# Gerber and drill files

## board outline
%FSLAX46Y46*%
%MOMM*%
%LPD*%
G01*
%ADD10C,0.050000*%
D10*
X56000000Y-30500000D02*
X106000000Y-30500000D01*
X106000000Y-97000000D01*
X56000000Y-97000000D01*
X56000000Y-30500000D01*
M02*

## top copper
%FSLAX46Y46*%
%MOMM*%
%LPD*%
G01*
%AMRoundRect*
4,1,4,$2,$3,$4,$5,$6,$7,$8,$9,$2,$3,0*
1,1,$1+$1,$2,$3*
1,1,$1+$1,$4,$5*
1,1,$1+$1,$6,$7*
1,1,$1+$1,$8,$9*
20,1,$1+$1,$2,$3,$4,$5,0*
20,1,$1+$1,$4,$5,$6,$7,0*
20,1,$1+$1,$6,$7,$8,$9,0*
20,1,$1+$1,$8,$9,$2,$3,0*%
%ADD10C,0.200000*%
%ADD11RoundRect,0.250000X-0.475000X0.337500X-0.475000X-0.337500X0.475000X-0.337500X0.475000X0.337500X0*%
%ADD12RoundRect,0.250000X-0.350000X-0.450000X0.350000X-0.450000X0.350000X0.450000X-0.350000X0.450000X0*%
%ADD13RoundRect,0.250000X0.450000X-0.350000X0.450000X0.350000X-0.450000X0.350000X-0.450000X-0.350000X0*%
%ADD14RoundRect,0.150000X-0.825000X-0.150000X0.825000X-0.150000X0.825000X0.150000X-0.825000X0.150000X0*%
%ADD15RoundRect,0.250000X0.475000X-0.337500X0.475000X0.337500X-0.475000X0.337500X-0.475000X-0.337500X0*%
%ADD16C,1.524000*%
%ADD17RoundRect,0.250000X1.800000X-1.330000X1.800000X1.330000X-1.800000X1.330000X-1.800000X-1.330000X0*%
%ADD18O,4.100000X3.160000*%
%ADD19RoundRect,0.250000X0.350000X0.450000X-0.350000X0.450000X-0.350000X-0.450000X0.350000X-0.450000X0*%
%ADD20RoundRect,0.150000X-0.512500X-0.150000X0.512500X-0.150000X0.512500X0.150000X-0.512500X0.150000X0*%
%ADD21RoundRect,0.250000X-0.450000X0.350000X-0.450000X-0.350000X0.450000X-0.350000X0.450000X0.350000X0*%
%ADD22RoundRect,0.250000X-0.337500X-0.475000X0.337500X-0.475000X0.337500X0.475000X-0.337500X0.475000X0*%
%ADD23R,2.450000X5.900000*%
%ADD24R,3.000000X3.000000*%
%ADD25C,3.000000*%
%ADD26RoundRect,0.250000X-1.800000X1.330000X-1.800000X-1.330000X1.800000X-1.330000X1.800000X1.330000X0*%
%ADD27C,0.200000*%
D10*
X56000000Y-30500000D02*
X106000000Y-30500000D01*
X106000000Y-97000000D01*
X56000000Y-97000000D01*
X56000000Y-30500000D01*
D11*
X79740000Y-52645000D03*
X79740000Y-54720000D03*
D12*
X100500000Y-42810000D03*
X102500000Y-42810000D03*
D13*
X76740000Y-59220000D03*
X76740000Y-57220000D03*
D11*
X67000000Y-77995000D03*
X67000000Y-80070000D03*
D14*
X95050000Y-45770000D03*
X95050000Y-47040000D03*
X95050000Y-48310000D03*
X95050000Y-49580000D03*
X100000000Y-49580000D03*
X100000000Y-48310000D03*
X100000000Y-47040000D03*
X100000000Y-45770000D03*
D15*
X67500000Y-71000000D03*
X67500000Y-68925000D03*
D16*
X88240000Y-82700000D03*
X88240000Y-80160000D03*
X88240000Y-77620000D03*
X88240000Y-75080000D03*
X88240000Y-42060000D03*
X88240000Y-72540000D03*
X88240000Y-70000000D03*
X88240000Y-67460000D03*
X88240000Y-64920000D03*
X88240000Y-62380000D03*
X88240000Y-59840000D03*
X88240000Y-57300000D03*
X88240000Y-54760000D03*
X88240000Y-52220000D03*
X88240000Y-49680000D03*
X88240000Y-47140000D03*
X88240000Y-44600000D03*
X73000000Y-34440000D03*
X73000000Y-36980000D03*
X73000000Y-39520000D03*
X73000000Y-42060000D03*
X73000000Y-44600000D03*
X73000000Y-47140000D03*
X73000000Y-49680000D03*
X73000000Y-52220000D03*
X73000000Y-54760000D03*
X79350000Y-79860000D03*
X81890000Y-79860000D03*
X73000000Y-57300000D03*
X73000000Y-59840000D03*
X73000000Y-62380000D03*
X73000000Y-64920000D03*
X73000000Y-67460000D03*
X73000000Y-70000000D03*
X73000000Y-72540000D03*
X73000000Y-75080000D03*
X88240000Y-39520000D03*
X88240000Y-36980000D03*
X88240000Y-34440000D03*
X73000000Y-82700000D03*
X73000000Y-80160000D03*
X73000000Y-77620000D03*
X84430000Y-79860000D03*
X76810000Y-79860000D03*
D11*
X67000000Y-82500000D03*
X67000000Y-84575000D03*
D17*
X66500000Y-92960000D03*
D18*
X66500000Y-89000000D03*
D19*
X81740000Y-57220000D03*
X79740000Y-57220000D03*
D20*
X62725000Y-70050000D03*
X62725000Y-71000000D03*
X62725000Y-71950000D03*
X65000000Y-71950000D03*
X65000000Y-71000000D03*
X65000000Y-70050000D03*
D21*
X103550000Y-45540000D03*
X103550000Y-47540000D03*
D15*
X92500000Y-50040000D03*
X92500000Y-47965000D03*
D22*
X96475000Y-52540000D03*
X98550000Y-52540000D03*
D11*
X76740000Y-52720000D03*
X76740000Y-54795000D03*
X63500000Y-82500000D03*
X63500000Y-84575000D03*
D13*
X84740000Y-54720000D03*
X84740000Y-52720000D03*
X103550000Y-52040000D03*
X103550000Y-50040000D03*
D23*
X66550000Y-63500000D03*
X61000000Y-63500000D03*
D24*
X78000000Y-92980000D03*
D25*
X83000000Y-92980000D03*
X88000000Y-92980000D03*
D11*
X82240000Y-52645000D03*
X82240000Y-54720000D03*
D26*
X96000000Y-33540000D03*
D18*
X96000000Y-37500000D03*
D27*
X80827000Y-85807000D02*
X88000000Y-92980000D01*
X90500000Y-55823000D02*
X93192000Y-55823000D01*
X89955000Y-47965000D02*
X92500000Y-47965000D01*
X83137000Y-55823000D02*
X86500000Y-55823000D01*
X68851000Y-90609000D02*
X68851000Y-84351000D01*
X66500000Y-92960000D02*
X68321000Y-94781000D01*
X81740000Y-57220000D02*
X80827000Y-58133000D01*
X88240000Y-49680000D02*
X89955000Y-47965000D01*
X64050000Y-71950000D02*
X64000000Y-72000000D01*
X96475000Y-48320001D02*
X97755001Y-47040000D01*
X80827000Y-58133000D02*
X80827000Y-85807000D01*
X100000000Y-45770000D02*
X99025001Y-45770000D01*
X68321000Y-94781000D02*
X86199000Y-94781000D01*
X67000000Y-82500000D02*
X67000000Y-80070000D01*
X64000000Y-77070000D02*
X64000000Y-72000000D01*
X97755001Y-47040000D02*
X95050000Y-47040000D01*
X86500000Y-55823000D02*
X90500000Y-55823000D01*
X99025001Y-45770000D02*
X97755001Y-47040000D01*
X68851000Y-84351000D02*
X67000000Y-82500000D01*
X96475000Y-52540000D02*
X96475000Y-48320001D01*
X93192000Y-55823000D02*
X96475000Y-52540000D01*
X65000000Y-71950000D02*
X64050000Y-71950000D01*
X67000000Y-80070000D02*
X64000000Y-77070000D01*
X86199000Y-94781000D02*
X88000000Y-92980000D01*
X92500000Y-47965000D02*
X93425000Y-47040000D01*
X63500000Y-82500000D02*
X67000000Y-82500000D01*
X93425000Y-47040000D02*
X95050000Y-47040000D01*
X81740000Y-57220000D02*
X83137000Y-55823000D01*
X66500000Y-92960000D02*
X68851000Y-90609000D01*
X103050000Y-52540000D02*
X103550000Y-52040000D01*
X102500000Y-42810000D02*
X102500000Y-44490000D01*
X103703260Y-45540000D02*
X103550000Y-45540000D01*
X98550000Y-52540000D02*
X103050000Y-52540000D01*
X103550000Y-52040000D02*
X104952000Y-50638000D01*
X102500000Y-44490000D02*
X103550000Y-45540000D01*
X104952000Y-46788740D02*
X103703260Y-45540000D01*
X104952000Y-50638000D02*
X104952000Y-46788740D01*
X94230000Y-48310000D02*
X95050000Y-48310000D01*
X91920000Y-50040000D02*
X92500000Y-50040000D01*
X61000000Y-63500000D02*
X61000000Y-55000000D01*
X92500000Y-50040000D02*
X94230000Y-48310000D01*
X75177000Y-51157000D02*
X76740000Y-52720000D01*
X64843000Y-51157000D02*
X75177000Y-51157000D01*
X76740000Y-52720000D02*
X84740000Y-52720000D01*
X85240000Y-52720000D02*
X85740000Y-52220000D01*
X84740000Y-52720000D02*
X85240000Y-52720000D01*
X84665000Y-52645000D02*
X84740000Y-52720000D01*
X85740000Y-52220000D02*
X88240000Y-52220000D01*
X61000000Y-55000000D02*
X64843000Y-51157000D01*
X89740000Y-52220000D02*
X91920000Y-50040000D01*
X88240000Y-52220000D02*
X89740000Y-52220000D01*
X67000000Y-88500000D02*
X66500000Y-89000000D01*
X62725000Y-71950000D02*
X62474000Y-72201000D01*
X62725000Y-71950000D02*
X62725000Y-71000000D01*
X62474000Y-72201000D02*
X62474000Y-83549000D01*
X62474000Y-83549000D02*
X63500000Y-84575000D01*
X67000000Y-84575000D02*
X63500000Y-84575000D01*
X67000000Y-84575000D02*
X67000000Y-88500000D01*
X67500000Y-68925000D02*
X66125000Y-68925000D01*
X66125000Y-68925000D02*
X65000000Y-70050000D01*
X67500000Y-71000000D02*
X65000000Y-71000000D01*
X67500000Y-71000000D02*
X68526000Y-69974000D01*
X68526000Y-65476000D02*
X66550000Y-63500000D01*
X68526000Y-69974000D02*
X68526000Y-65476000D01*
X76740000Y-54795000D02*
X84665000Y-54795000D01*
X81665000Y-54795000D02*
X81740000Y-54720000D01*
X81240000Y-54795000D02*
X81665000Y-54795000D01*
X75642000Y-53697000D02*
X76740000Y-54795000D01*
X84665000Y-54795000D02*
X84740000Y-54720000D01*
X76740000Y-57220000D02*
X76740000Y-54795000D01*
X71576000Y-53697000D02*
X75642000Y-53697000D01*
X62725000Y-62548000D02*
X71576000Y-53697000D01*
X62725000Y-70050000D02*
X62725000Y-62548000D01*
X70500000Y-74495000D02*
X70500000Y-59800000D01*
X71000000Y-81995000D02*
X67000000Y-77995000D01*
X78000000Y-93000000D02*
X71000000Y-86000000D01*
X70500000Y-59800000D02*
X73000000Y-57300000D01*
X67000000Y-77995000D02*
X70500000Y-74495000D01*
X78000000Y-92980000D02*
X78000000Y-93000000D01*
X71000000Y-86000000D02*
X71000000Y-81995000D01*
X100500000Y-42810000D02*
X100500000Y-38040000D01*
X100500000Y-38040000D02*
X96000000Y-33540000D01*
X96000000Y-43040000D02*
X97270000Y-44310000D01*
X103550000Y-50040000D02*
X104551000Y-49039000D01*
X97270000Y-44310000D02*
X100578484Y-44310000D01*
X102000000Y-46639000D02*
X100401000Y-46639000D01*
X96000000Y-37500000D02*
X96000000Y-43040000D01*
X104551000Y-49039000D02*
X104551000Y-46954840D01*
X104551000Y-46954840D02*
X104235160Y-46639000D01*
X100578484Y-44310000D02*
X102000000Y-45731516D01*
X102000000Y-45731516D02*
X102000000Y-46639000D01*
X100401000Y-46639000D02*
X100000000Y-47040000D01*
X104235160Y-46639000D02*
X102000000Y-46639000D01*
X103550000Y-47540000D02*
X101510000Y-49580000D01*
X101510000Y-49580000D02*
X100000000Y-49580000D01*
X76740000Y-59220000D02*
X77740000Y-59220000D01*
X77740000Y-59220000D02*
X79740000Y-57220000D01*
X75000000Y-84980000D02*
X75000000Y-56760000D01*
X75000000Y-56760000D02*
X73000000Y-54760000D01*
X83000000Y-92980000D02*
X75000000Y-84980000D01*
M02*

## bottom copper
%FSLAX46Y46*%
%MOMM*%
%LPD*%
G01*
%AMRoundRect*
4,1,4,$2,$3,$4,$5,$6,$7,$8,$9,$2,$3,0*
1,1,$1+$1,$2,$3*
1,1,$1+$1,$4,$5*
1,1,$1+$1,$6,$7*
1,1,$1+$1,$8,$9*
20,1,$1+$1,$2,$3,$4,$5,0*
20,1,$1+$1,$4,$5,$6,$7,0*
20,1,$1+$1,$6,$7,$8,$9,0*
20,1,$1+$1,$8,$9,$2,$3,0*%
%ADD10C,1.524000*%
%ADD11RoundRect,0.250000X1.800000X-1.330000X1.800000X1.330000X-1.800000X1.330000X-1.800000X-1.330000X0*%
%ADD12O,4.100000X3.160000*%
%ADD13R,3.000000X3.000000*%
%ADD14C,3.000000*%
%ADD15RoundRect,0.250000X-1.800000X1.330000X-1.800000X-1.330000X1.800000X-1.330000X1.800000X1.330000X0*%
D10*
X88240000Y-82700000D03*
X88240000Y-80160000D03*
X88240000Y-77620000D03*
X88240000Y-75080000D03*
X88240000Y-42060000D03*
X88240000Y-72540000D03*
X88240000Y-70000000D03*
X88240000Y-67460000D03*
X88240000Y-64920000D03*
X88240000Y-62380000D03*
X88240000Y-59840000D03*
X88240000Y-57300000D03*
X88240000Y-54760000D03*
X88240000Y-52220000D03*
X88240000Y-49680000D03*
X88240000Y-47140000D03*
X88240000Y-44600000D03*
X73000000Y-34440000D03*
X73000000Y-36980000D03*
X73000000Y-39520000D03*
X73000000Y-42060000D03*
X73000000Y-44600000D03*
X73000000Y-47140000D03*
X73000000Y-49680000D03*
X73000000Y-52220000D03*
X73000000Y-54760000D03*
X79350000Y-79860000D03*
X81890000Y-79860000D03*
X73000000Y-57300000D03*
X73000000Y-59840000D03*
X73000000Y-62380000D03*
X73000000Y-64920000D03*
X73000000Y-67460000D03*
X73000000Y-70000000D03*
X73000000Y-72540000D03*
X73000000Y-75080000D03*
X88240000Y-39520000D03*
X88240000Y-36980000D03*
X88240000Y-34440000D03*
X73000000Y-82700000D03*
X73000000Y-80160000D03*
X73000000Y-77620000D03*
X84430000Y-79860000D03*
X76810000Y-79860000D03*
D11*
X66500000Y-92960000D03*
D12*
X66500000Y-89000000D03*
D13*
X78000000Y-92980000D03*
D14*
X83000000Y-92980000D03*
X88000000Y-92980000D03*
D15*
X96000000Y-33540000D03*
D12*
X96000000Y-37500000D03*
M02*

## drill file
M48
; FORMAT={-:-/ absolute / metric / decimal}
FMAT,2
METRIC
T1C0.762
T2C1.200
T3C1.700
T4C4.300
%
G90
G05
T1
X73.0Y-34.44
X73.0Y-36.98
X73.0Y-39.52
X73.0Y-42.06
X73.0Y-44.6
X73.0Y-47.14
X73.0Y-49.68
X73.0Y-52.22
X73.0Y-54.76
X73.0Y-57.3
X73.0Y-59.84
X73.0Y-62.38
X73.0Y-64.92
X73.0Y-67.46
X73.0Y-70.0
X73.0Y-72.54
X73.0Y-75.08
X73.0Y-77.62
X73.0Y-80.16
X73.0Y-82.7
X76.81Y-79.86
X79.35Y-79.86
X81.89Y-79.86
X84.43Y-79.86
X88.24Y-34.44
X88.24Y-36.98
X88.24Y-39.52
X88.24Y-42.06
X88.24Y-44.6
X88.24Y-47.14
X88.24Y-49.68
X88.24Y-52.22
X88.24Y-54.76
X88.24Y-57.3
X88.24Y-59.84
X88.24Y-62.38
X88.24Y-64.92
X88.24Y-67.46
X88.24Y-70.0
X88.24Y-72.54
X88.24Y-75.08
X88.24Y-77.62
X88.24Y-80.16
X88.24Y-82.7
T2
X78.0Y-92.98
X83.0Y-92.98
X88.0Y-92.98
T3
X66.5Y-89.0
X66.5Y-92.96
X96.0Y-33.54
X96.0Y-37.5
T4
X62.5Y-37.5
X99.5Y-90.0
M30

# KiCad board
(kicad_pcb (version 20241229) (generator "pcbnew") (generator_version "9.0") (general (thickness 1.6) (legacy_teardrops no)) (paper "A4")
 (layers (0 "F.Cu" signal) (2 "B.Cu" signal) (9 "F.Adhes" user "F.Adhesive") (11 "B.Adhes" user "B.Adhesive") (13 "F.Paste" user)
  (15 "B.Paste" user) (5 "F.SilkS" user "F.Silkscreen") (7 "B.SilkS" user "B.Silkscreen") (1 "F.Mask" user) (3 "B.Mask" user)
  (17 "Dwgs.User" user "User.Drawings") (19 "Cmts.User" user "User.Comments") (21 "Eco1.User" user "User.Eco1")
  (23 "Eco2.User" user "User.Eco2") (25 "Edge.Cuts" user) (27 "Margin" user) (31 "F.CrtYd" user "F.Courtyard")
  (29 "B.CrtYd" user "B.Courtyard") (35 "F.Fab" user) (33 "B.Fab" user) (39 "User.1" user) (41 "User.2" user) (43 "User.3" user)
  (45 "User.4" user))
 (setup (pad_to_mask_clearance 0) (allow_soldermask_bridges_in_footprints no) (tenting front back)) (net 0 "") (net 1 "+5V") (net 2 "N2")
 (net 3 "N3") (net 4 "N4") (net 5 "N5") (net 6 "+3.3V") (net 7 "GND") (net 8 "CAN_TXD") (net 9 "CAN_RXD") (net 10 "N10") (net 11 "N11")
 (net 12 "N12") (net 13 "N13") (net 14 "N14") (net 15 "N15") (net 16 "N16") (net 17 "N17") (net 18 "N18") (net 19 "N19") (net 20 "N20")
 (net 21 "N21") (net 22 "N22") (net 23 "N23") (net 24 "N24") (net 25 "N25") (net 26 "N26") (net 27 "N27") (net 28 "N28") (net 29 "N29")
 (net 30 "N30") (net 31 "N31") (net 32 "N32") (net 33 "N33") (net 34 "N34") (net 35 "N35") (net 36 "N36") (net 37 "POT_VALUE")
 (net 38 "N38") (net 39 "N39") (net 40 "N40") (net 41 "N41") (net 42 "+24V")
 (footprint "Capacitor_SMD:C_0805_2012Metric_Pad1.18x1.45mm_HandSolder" (layer "F.Cu") (at 79.74 53.6825 -90)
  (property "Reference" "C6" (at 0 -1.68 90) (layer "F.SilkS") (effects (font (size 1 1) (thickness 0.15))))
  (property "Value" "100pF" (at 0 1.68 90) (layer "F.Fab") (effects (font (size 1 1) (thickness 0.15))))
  (pad "1" smd roundrect (at -1.0375 0 270) (size 1.175 1.45) (layers "F.Cu" "F.Mask" "F.Paste") (roundrect_rratio 0.212766) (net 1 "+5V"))
  (pad "2" smd roundrect (at 1.0375 0 270) (size 1.175 1.45) (layers "F.Cu" "F.Mask" "F.Paste") (roundrect_rratio 0.212766) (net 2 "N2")))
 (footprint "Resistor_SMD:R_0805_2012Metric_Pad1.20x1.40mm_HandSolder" (layer "F.Cu") (at 101.5 42.81)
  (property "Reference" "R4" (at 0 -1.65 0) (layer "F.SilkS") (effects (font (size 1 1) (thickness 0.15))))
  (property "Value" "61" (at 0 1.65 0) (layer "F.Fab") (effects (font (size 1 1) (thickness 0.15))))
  (pad "1" smd roundrect (at -1 0) (size 1.2 1.4) (layers "F.Cu" "F.Mask" "F.Paste") (roundrect_rratio 0.208333) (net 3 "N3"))
  (pad "2" smd roundrect (at 1 0) (size 1.2 1.4) (layers "F.Cu" "F.Mask" "F.Paste") (roundrect_rratio 0.208333) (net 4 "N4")))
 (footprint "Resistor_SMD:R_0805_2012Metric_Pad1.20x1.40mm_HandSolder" (layer "F.Cu") (at 76.74 58.22 90)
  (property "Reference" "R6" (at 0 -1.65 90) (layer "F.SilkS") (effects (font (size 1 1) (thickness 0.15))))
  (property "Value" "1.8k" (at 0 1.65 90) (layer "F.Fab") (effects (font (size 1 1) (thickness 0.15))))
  (pad "1" smd roundrect (at -1 0 90) (size 1.2 1.4) (layers "F.Cu" "F.Mask" "F.Paste") (roundrect_rratio 0.208333) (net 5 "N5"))
  (pad "2" smd roundrect (at 1 0 90) (size 1.2 1.4) (layers "F.Cu" "F.Mask" "F.Paste") (roundrect_rratio 0.208333) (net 2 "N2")))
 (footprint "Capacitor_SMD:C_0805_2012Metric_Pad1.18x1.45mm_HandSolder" (layer "F.Cu") (at 67 79.0325 -90)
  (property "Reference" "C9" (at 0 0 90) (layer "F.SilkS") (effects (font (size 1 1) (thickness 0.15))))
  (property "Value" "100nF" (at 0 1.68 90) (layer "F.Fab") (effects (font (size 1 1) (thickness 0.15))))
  (pad "1" smd roundrect (at -1.0375 0 270) (size 1.175 1.45) (layers "F.Cu" "F.Mask" "F.Paste") (roundrect_rratio 0.212766) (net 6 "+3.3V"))
  (pad "2" smd roundrect (at 1.0375 0 270) (size 1.175 1.45) (layers "F.Cu" "F.Mask" "F.Paste") (roundrect_rratio 0.212766) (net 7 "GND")))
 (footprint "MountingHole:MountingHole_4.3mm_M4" (layer "F.Cu") (at 62.5 37.5)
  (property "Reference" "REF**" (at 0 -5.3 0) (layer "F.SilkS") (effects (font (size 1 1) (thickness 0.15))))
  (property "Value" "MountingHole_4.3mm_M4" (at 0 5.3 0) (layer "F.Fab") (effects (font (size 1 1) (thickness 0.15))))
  (pad "" np_thru_hole circle (at 0 0) (size 4.3 4.3) (drill 4.3) (layers "*.Cu" "*.Mask")))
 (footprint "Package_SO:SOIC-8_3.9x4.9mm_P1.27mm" (layer "F.Cu") (at 97.525 47.675)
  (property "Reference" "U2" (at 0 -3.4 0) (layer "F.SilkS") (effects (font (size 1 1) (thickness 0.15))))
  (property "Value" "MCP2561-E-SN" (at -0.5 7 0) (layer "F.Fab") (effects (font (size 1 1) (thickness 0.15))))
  (pad "1" smd roundrect (at -2.475 -1.905) (size 1.95 0.6) (layers "F.Cu" "F.Mask" "F.Paste") (roundrect_rratio 0.25) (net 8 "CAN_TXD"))
  (pad "2" smd roundrect (at -2.475 -0.635) (size 1.95 0.6) (layers "F.Cu" "F.Mask" "F.Paste") (roundrect_rratio 0.25) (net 7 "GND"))
  (pad "3" smd roundrect (at -2.475 0.635) (size 1.95 0.6) (layers "F.Cu" "F.Mask" "F.Paste") (roundrect_rratio 0.25) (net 1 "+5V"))
  (pad "4" smd roundrect (at -2.475 1.905) (size 1.95 0.6) (layers "F.Cu" "F.Mask" "F.Paste") (roundrect_rratio 0.25) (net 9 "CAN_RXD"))
  (pad "5" smd roundrect (at 2.475 1.905) (size 1.95 0.6) (layers "F.Cu" "F.Mask" "F.Paste") (roundrect_rratio 0.25) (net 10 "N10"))
  (pad "6" smd roundrect (at 2.475 0.635) (size 1.95 0.6) (layers "F.Cu" "F.Mask" "F.Paste") (roundrect_rratio 0.25) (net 3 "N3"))
  (pad "7" smd roundrect (at 2.475 -0.635) (size 1.95 0.6) (layers "F.Cu" "F.Mask" "F.Paste") (roundrect_rratio 0.25) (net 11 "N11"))
  (pad "8" smd roundrect (at 2.475 -1.905) (size 1.95 0.6) (layers "F.Cu" "F.Mask" "F.Paste") (roundrect_rratio 0.25) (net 7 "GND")))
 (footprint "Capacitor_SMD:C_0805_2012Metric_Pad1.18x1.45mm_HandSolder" (layer "F.Cu") (at 67.5 69.9625 90)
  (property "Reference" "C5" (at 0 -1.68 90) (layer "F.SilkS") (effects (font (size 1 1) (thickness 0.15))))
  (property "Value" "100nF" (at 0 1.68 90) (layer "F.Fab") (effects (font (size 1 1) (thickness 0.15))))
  (pad "1" smd roundrect (at -1.0375 0 90) (size 1.175 1.45) (layers "F.Cu" "F.Mask" "F.Paste") (roundrect_rratio 0.212766) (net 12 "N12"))
  (pad "2" smd roundrect (at 1.0375 0 90) (size 1.175 1.45) (layers "F.Cu" "F.Mask" "F.Paste") (roundrect_rratio 0.212766) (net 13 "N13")))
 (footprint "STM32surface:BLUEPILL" (layer "F.Cu") (at 80.62 61.11 180)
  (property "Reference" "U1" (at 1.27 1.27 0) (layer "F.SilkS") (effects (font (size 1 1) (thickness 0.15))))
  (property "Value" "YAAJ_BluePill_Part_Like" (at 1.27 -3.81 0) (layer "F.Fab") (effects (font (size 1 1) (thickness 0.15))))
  (pad "1" thru_hole circle (at -7.62 -21.59 180) (size 1.524 1.524) (drill 0.762) (layers "*.Cu" "*.Mask") (remove_unused_layers no)
   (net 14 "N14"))
  (pad "2" thru_hole circle (at -7.62 -19.05 180) (size 1.524 1.524) (drill 0.762) (layers "*.Cu" "*.Mask") (remove_unused_layers no)
   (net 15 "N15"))
  (pad "3" thru_hole circle (at -7.62 -16.51 180) (size 1.524 1.524) (drill 0.762) (layers "*.Cu" "*.Mask") (remove_unused_layers no)
   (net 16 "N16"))
  (pad "4" thru_hole circle (at -7.62 -13.97 180) (size 1.524 1.524) (drill 0.762) (layers "*.Cu" "*.Mask") (remove_unused_layers no)
   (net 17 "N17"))
  (pad "7" thru_hole circle (at -7.62 19.05 180) (size 1.524 1.524) (drill 0.762) (layers "*.Cu" "*.Mask") (remove_unused_layers no)
   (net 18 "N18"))
  (pad "10" thru_hole circle (at -7.62 -11.43 180) (size 1.524 1.524) (drill 0.762) (layers "*.Cu" "*.Mask") (remove_unused_layers no)
   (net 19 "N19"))
  (pad "11" thru_hole circle (at -7.62 -8.89 180) (size 1.524 1.524) (drill 0.762) (layers "*.Cu" "*.Mask") (remove_unused_layers no)
   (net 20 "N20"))
  (pad "12" thru_hole circle (at -7.62 -6.35 180) (size 1.524 1.524) (drill 0.762) (layers "*.Cu" "*.Mask") (remove_unused_layers no)
   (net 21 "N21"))
  (pad "13" thru_hole circle (at -7.62 -3.81 180) (size 1.524 1.524) (drill 0.762) (layers "*.Cu" "*.Mask") (remove_unused_layers no)
   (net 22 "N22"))
  (pad "14" thru_hole circle (at -7.62 -1.27 180) (size 1.524 1.524) (drill 0.762) (layers "*.Cu" "*.Mask") (remove_unused_layers no)
   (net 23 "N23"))
  (pad "15" thru_hole circle (at -7.62 1.27 180) (size 1.524 1.524) (drill 0.762) (layers "*.Cu" "*.Mask") (remove_unused_layers no)
   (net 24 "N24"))
  (pad "16" thru_hole circle (at -7.62 3.81 180) (size 1.524 1.524) (drill 0.762) (layers "*.Cu" "*.Mask") (remove_unused_layers no)
   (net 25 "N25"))
  (pad "17" thru_hole circle (at -7.62 6.35 180) (size 1.524 1.524) (drill 0.762) (layers "*.Cu" "*.Mask") (remove_unused_layers no)
   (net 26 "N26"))
  (pad "18" thru_hole circle (at -7.62 8.89 180) (size 1.524 1.524) (drill 0.762) (layers "*.Cu" "*.Mask") (remove_unused_layers no)
   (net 1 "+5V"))
  (pad "19" thru_hole circle (at -7.62 11.43 180) (size 1.524 1.524) (drill 0.762) (layers "*.Cu" "*.Mask") (remove_unused_layers no)
   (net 7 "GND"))
  (pad "21" thru_hole circle (at -7.62 13.97 180) (size 1.524 1.524) (drill 0.762) (layers "*.Cu" "*.Mask") (remove_unused_layers no)
   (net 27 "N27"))
  (pad "22" thru_hole circle (at -7.62 16.51 180) (size 1.524 1.524) (drill 0.762) (layers "*.Cu" "*.Mask") (remove_unused_layers no)
   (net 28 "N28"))
  (pad "25" thru_hole circle (at 7.62 26.67 180) (size 1.524 1.524) (drill 0.762) (layers "*.Cu" "*.Mask") (remove_unused_layers no)
   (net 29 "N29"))
  (pad "26" thru_hole circle (at 7.62 24.13 180) (size 1.524 1.524) (drill 0.762) (layers "*.Cu" "*.Mask") (remove_unused_layers no)
   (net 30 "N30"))
  (pad "27" thru_hole circle (at 7.62 21.59 180) (size 1.524 1.524) (drill 0.762) (layers "*.Cu" "*.Mask") (remove_unused_layers no)
   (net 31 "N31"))
  (pad "28" thru_hole circle (at 7.62 19.05 180) (size 1.524 1.524) (drill 0.762) (layers "*.Cu" "*.Mask") (remove_unused_layers no)
   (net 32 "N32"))
  (pad "29" thru_hole circle (at 7.62 16.51 180) (size 1.524 1.524) (drill 0.762) (layers "*.Cu" "*.Mask") (remove_unused_layers no)
   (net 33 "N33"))
  (pad "30" thru_hole circle (at 7.62 13.97 180) (size 1.524 1.524) (drill 0.762) (layers "*.Cu" "*.Mask") (remove_unused_layers no)
   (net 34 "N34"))
  (pad "31" thru_hole circle (at 7.62 11.43 180) (size 1.524 1.524) (drill 0.762) (layers "*.Cu" "*.Mask") (remove_unused_layers no)
   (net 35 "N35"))
  (pad "32" thru_hole circle (at 7.62 8.89 180) (size 1.524 1.524) (drill 0.762) (layers "*.Cu" "*.Mask") (remove_unused_layers no)
   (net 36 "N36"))
  (pad "33" thru_hole circle (at 7.62 6.35 180) (size 1.524 1.524) (drill 0.762) (layers "*.Cu" "*.Mask") (remove_unused_layers no)
   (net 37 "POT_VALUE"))
  (pad "34" thru_hole circle (at 1.27 -18.75 180) (size 1.524 1.524) (drill 0.762) (layers "*.Cu" "*.Mask") (remove_unused_layers no)
   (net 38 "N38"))
  (pad "37" thru_hole circle (at -1.27 -18.75 180) (size 1.524 1.524) (drill 0.762) (layers "*.Cu" "*.Mask") (remove_unused_layers no)
   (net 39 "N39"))
  (pad "38" thru_hole circle (at 7.62 3.81 180) (size 1.524 1.524) (drill 0.762) (layers "*.Cu" "*.Mask") (remove_unused_layers no)
   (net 6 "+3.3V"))
  (pad "39" thru_hole circle (at 7.62 1.27 180) (size 1.524 1.524) (drill 0.762) (layers "*.Cu" "*.Mask") (remove_unused_layers no)
   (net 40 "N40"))
  (pad "40" thru_hole circle (at 7.62 -1.27 180) (size 1.524 1.524) (drill 0.762) (layers "*.Cu" "*.Mask") (remove_unused_layers no)
   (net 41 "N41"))
  (pad "41" thru_hole circle (at 7.62 -3.81 180) (size 1.524 1.524) (drill 0.762) (layers "*.Cu" "*.Mask") (remove_unused_layers no))
  (pad "42" thru_hole circle (at 7.62 -6.35 180) (size 1.524 1.524) (drill 0.762) (layers "*.Cu" "*.Mask") (remove_unused_layers no))
  (pad "43" thru_hole circle (at 7.62 -8.89 180) (size 1.524 1.524) (drill 0.762) (layers "*.Cu" "*.Mask") (remove_unused_layers no))
  (pad "45" thru_hole circle (at 7.62 -11.43 180) (size 1.524 1.524) (drill 0.762) (layers "*.Cu" "*.Mask") (remove_unused_layers no))
  (pad "46" thru_hole circle (at 7.62 -13.97 180) (size 1.524 1.524) (drill 0.762) (layers "*.Cu" "*.Mask") (remove_unused_layers no))
  (pad "70" thru_hole circle (at -7.62 21.59 180) (size 1.524 1.524) (drill 0.762) (layers "*.Cu" "*.Mask") (remove_unused_layers no))
  (pad "71" thru_hole circle (at -7.62 24.13 180) (size 1.524 1.524) (drill 0.762) (layers "*.Cu" "*.Mask") (remove_unused_layers no))
  (pad "72" thru_hole circle (at -7.62 26.67 180) (size 1.524 1.524) (drill 0.762) (layers "*.Cu" "*.Mask") (remove_unused_layers no))
  (pad "73" thru_hole circle (at 7.62 -21.59 180) (size 1.524 1.524) (drill 0.762) (layers "*.Cu" "*.Mask") (remove_unused_layers no))
  (pad "74" thru_hole circle (at 7.62 -19.05 180) (size 1.524 1.524) (drill 0.762) (layers "*.Cu" "*.Mask") (remove_unused_layers no))
  (pad "75" thru_hole circle (at 7.62 -16.51 180) (size 1.524 1.524) (drill 0.762) (layers "*.Cu" "*.Mask") (remove_unused_layers no))
  (pad "76" thru_hole circle (at -3.81 -18.75 180) (size 1.524 1.524) (drill 0.762) (layers "*.Cu" "*.Mask") (remove_unused_layers no))
  (pad "77" thru_hole circle (at 3.81 -18.75 180) (size 1.524 1.524) (drill 0.762) (layers "*.Cu" "*.Mask") (remove_unused_layers no)))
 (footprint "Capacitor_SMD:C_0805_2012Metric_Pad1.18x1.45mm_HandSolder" (layer "F.Cu") (at 67 83.5375 -90)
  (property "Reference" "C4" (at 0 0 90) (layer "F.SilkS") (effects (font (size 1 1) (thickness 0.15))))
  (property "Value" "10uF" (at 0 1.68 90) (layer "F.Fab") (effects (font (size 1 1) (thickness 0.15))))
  (pad "1" smd roundrect (at -1.0375 0 270) (size 1.175 1.45) (layers "F.Cu" "F.Mask" "F.Paste") (roundrect_rratio 0.212766) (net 7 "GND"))
  (pad "2" smd roundrect (at 1.0375 0 270) (size 1.175 1.45) (layers "F.Cu" "F.Mask" "F.Paste") (roundrect_rratio 0.212766) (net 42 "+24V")))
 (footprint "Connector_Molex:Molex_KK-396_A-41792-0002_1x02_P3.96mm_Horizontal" (layer "F.Cu") (at 66.5 92.96 90)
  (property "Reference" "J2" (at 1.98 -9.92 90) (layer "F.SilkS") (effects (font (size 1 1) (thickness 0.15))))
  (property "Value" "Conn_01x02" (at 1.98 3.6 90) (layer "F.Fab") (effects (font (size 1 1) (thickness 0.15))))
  (pad "1" thru_hole roundrect (at 0 0 90) (size 3.16 4.1) (drill 1.7) (layers "*.Cu" "*.Mask") (remove_unused_layers no)
   (roundrect_rratio 0.079114) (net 7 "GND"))
  (pad "2" thru_hole oval (at 3.96 0 90) (size 3.16 4.1) (drill 1.7) (layers "*.Cu" "*.Mask") (remove_unused_layers no) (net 42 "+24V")))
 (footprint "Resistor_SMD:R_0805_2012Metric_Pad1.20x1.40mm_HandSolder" (layer "F.Cu") (at 80.74 57.22 180)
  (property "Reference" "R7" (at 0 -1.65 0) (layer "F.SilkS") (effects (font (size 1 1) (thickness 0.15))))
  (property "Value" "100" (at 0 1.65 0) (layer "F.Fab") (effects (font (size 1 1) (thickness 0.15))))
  (pad "1" smd roundrect (at -1 0 180) (size 1.2 1.4) (layers "F.Cu" "F.Mask" "F.Paste") (roundrect_rratio 0.208333) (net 7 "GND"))
  (pad "2" smd roundrect (at 1 0 180) (size 1.2 1.4) (layers "F.Cu" "F.Mask" "F.Paste") (roundrect_rratio 0.208333) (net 5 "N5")))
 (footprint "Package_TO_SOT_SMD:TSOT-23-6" (layer "F.Cu") (at 63.8625 71)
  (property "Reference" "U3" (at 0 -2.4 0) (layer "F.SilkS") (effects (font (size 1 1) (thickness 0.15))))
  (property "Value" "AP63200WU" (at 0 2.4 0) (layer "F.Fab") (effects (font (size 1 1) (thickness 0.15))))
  (pad "1" smd roundrect (at -1.1375 -0.95) (size 1.325 0.6) (layers "F.Cu" "F.Mask" "F.Paste") (roundrect_rratio 0.25) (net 2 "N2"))
  (pad "2" smd roundrect (at -1.1375 0) (size 1.325 0.6) (layers "F.Cu" "F.Mask" "F.Paste") (roundrect_rratio 0.25) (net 42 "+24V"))
  (pad "3" smd roundrect (at -1.1375 0.95) (size 1.325 0.6) (layers "F.Cu" "F.Mask" "F.Paste") (roundrect_rratio 0.25) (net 42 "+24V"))
  (pad "4" smd roundrect (at 1.1375 0.95) (size 1.325 0.6) (layers "F.Cu" "F.Mask" "F.Paste") (roundrect_rratio 0.25) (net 7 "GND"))
  (pad "5" smd roundrect (at 1.1375 0) (size 1.325 0.6) (layers "F.Cu" "F.Mask" "F.Paste") (roundrect_rratio 0.25) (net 12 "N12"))
  (pad "6" smd roundrect (at 1.1375 -0.95) (size 1.325 0.6) (layers "F.Cu" "F.Mask" "F.Paste") (roundrect_rratio 0.25) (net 13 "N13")))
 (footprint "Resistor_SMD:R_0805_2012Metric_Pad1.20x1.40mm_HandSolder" (layer "F.Cu") (at 103.55 46.54 -90)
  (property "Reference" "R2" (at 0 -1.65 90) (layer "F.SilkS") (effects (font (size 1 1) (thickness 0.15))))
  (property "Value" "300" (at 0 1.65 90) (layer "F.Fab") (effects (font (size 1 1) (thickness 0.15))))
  (pad "1" smd roundrect (at -1 0 270) (size 1.2 1.4) (layers "F.Cu" "F.Mask" "F.Paste") (roundrect_rratio 0.208333) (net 4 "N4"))
  (pad "2" smd roundrect (at 1 0 270) (size 1.2 1.4) (layers "F.Cu" "F.Mask" "F.Paste") (roundrect_rratio 0.208333) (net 10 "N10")))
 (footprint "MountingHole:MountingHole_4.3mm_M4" (layer "F.Cu") (at 99.5 90)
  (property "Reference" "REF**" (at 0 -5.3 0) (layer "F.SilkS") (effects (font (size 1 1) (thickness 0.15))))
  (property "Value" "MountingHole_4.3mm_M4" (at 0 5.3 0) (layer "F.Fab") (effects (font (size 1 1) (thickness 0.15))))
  (pad "" np_thru_hole circle (at 0 0) (size 4.3 4.3) (drill 4.3) (layers "*.Cu" "*.Mask")))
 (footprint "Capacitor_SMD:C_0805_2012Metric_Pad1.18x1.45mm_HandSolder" (layer "F.Cu") (at 92.5 49.0025 90)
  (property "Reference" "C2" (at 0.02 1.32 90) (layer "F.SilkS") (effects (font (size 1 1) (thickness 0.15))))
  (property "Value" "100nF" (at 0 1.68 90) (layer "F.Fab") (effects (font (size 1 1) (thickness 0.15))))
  (pad "1" smd roundrect (at -1.0375 0 90) (size 1.175 1.45) (layers "F.Cu" "F.Mask" "F.Paste") (roundrect_rratio 0.212766) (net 1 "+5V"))
  (pad "2" smd roundrect (at 1.0375 0 90) (size 1.175 1.45) (layers "F.Cu" "F.Mask" "F.Paste") (roundrect_rratio 0.212766) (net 7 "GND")))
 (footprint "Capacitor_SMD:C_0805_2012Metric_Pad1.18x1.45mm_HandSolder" (layer "F.Cu") (at 97.5125 52.54)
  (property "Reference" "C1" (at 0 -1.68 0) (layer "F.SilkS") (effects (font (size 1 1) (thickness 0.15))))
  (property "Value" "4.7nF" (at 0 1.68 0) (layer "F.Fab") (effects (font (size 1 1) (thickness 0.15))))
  (pad "1" smd roundrect (at -1.0375 0) (size 1.175 1.45) (layers "F.Cu" "F.Mask" "F.Paste") (roundrect_rratio 0.212766) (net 7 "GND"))
  (pad "2" smd roundrect (at 1.0375 0) (size 1.175 1.45) (layers "F.Cu" "F.Mask" "F.Paste") (roundrect_rratio 0.212766) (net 4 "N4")))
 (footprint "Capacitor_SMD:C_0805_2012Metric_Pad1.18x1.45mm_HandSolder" (layer "F.Cu") (at 76.74 53.7575 -90)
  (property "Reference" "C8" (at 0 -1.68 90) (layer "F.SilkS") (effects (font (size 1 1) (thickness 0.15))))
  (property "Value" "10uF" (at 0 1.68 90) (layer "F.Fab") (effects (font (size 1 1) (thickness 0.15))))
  (pad "1" smd roundrect (at -1.0375 0 270) (size 1.175 1.45) (layers "F.Cu" "F.Mask" "F.Paste") (roundrect_rratio 0.212766) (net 1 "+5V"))
  (pad "2" smd roundrect (at 1.0375 0 270) (size 1.175 1.45) (layers "F.Cu" "F.Mask" "F.Paste") (roundrect_rratio 0.212766) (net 2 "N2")))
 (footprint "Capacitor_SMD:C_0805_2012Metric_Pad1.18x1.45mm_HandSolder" (layer "F.Cu") (at 63.5 83.5375 -90)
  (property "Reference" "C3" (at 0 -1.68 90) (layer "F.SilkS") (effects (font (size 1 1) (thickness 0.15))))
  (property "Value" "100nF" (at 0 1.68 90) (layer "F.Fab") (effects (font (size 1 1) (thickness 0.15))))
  (pad "1" smd roundrect (at -1.0375 0 270) (size 1.175 1.45) (layers "F.Cu" "F.Mask" "F.Paste") (roundrect_rratio 0.212766) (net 7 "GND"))
  (pad "2" smd roundrect (at 1.0375 0 270) (size 1.175 1.45) (layers "F.Cu" "F.Mask" "F.Paste") (roundrect_rratio 0.212766) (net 42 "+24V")))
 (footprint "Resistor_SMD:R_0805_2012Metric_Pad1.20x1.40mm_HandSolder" (layer "F.Cu") (at 84.74 53.72 90)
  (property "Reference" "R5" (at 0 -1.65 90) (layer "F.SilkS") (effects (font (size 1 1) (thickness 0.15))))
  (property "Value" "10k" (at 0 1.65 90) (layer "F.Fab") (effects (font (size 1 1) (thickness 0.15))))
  (pad "1" smd roundrect (at -1 0 90) (size 1.2 1.4) (layers "F.Cu" "F.Mask" "F.Paste") (roundrect_rratio 0.208333) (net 2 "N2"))
  (pad "2" smd roundrect (at 1 0 90) (size 1.2 1.4) (layers "F.Cu" "F.Mask" "F.Paste") (roundrect_rratio 0.208333) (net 1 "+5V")))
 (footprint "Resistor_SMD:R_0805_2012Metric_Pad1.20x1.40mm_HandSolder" (layer "F.Cu") (at 103.55 51.04 90)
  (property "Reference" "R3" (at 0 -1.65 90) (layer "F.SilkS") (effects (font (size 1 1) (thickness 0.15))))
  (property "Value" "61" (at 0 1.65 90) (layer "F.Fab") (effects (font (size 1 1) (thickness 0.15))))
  (pad "1" smd roundrect (at -1 0 90) (size 1.2 1.4) (layers "F.Cu" "F.Mask" "F.Paste") (roundrect_rratio 0.208333) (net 4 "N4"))
  (pad "2" smd roundrect (at 1 0 90) (size 1.2 1.4) (layers "F.Cu" "F.Mask" "F.Paste") (roundrect_rratio 0.208333) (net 11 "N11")))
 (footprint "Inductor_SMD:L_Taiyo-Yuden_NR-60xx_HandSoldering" (layer "F.Cu") (at 63.775 63.5 180)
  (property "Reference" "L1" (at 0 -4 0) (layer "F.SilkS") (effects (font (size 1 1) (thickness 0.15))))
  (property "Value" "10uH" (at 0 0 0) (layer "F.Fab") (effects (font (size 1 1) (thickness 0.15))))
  (pad "1" smd rect (at -2.775 0 180) (size 2.45 5.9) (layers "F.Cu" "F.Mask" "F.Paste") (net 12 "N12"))
  (pad "2" smd rect (at 2.775 0 180) (size 2.45 5.9) (layers "F.Cu" "F.Mask" "F.Paste") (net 1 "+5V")))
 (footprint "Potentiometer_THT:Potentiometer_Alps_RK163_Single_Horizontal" (layer "F.Cu") (at 78 92.98 90)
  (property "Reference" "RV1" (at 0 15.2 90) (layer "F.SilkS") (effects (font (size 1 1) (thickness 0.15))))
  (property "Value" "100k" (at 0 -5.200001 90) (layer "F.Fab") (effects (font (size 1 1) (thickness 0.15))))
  (pad "1" thru_hole rect (at 0 0 270) (size 3 3) (drill 1.2) (layers "*.Cu" "*.Mask") (remove_unused_layers no) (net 6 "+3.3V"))
  (pad "2" thru_hole circle (at 0 5 270) (size 3 3) (drill 1.2) (layers "*.Cu" "*.Mask") (remove_unused_layers no) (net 37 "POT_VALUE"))
  (pad "3" thru_hole circle (at 0 10 270) (size 3 3) (drill 1.2) (layers "*.Cu" "*.Mask") (remove_unused_layers no) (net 7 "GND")))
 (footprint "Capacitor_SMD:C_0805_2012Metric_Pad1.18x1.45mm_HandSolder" (layer "F.Cu") (at 82.24 53.6825 -90)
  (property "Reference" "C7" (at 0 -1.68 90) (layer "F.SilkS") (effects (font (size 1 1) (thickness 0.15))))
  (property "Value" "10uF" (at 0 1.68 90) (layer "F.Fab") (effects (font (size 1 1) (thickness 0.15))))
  (pad "1" smd roundrect (at -1.0375 0 270) (size 1.175 1.45) (layers "F.Cu" "F.Mask" "F.Paste") (roundrect_rratio 0.212766) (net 1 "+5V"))
  (pad "2" smd roundrect (at 1.0375 0 270) (size 1.175 1.45) (layers "F.Cu" "F.Mask" "F.Paste") (roundrect_rratio 0.212766) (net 2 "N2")))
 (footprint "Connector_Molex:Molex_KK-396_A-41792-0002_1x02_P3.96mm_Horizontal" (layer "F.Cu") (at 96 33.54 -90)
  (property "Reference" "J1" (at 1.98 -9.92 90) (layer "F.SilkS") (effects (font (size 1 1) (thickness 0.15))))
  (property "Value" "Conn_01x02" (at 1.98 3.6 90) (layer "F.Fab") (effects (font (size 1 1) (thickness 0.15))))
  (pad "1" thru_hole roundrect (at 0 0 270) (size 3.16 4.1) (drill 1.7) (layers "*.Cu" "*.Mask") (remove_unused_layers no)
   (roundrect_rratio 0.079114) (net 3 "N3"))
  (pad "2" thru_hole oval (at 3.96 0 270) (size 3.16 4.1) (drill 1.7) (layers "*.Cu" "*.Mask") (remove_unused_layers no) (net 11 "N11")))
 (gr_rect (start 56 30.5) (end 106 97) (stroke (width 0.2) (type default)) (fill no) (layer "F.Cu"))
 (gr_rect (start 56 30.5) (end 106 97) (stroke (width 0.05) (type default)) (fill no) (layer "Edge.Cuts"))
 (segment (start 80.827 85.807) (end 88 92.98) (width 0.2) (layer "F.Cu") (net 7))
 (segment (start 90.5 55.823) (end 93.192 55.823) (width 0.2) (layer "F.Cu") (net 7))
 (segment (start 89.955 47.965) (end 92.5 47.965) (width 0.2) (layer "F.Cu") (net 7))
 (segment (start 83.137 55.823) (end 86.5 55.823) (width 0.2) (layer "F.Cu") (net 7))
 (segment (start 68.851 90.609) (end 68.851 84.351) (width 0.2) (layer "F.Cu") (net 7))
 (segment (start 66.5 92.96) (end 68.321 94.781) (width 0.2) (layer "F.Cu") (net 7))
 (segment (start 81.74 57.22) (end 80.827 58.133) (width 0.2) (layer "F.Cu") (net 7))
 (segment (start 88.24 49.68) (end 89.955 47.965) (width 0.2) (layer "F.Cu") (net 7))
 (segment (start 64.05 71.95) (end 64 72) (width 0.2) (layer "F.Cu") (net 7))
 (segment (start 96.475 48.320001) (end 97.755001 47.04) (width 0.2) (layer "F.Cu") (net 7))
 (segment (start 80.827 58.133) (end 80.827 85.807) (width 0.2) (layer "F.Cu") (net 7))
 (segment (start 100 45.77) (end 99.025001 45.77) (width 0.2) (layer "F.Cu") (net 7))
 (segment (start 68.321 94.781) (end 86.199 94.781) (width 0.2) (layer "F.Cu") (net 7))
 (segment (start 67 82.5) (end 67 80.07) (width 0.2) (layer "F.Cu") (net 7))
 (segment (start 64 77.07) (end 64 72) (width 0.2) (layer "F.Cu") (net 7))
 (segment (start 97.755001 47.04) (end 95.05 47.04) (width 0.2) (layer "F.Cu") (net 7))
 (segment (start 86.5 55.823) (end 90.5 55.823) (width 0.2) (layer "F.Cu") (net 7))
 (segment (start 99.025001 45.77) (end 97.755001 47.04) (width 0.2) (layer "F.Cu") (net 7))
 (segment (start 68.851 84.351) (end 67 82.5) (width 0.2) (layer "F.Cu") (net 7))
 (segment (start 96.475 52.54) (end 96.475 48.320001) (width 0.2) (layer "F.Cu") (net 7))
 (segment (start 93.192 55.823) (end 96.475 52.54) (width 0.2) (layer "F.Cu") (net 7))
 (segment (start 65 71.95) (end 64.05 71.95) (width 0.2) (layer "F.Cu") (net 7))
 (segment (start 67 80.07) (end 64 77.07) (width 0.2) (layer "F.Cu") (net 7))
 (segment (start 86.199 94.781) (end 88 92.98) (width 0.2) (layer "F.Cu") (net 7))
 (segment (start 92.5 47.965) (end 93.425 47.04) (width 0.2) (layer "F.Cu") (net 7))
 (segment (start 63.5 82.5) (end 67 82.5) (width 0.2) (layer "F.Cu") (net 7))
 (segment (start 93.425 47.04) (end 95.05 47.04) (width 0.2) (layer "F.Cu") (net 7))
 (segment (start 81.74 57.22) (end 83.137 55.823) (width 0.2) (layer "F.Cu") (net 7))
 (segment (start 66.5 92.96) (end 68.851 90.609) (width 0.2) (layer "F.Cu") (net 7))
 (segment (start 103.05 52.54) (end 103.55 52.04) (width 0.2) (layer "F.Cu") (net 4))
 (segment (start 102.5 42.81) (end 102.5 44.49) (width 0.2) (layer "F.Cu") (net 4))
 (segment (start 103.70326 45.54) (end 103.55 45.54) (width 0.2) (layer "F.Cu") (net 4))
 (segment (start 98.55 52.54) (end 103.05 52.54) (width 0.2) (layer "F.Cu") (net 4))
 (segment (start 103.55 52.04) (end 104.952 50.638) (width 0.2) (layer "F.Cu") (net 4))
 (segment (start 102.5 44.49) (end 103.55 45.54) (width 0.2) (layer "F.Cu") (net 4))
 (segment (start 104.952 46.78874) (end 103.70326 45.54) (width 0.2) (layer "F.Cu") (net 4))
 (segment (start 104.952 50.638) (end 104.952 46.78874) (width 0.2) (layer "F.Cu") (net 4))
 (segment (start 94.23 48.31) (end 95.05 48.31) (width 0.2) (layer "F.Cu") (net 1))
 (segment (start 91.92 50.04) (end 92.5 50.04) (width 0.2) (layer "F.Cu") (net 1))
 (segment (start 61 63.5) (end 61 55) (width 0.2) (layer "F.Cu") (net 1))
 (segment (start 92.5 50.04) (end 94.23 48.31) (width 0.2) (layer "F.Cu") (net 1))
 (segment (start 75.177 51.157) (end 76.74 52.72) (width 0.2) (layer "F.Cu") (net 1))
 (segment (start 64.843 51.157) (end 75.177 51.157) (width 0.2) (layer "F.Cu") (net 1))
 (segment (start 76.74 52.72) (end 84.74 52.72) (width 0.2) (layer "F.Cu") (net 1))
 (segment (start 85.24 52.72) (end 85.74 52.22) (width 0.2) (layer "F.Cu") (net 1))
 (segment (start 84.74 52.72) (end 85.24 52.72) (width 0.2) (layer "F.Cu") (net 1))
 (segment (start 84.665 52.645) (end 84.74 52.72) (width 0.2) (layer "F.Cu") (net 1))
 (segment (start 85.74 52.22) (end 88.24 52.22) (width 0.2) (layer "F.Cu") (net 1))
 (segment (start 61 55) (end 64.843 51.157) (width 0.2) (layer "F.Cu") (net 1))
 (segment (start 89.74 52.22) (end 91.92 50.04) (width 0.2) (layer "F.Cu") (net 1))
 (segment (start 88.24 52.22) (end 89.74 52.22) (width 0.2) (layer "F.Cu") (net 1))
 (segment (start 67 88.5) (end 66.5 89) (width 0.2) (layer "F.Cu") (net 42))
 (segment (start 62.725 71.95) (end 62.474 72.201) (width 0.2) (layer "F.Cu") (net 42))
 (segment (start 62.725 71.95) (end 62.725 71) (width 0.2) (layer "F.Cu") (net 42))
 (segment (start 62.474 72.201) (end 62.474 83.549) (width 0.2) (layer "F.Cu") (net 42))
 (segment (start 62.474 83.549) (end 63.5 84.575) (width 0.2) (layer "F.Cu") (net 42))
 (segment (start 67 84.575) (end 63.5 84.575) (width 0.2) (layer "F.Cu") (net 42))
 (segment (start 67 84.575) (end 67 88.5) (width 0.2) (layer "F.Cu") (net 42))
 (segment (start 67.5 68.925) (end 66.125 68.925) (width 0.2) (layer "F.Cu") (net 13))
 (segment (start 66.125 68.925) (end 65 70.05) (width 0.2) (layer "F.Cu") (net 13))
 (segment (start 67.5 71) (end 65 71) (width 0.2) (layer "F.Cu") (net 12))
 (segment (start 67.5 71) (end 68.526 69.974) (width 0.2) (layer "F.Cu") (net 12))
 (segment (start 68.526 65.476) (end 66.55 63.5) (width 0.2) (layer "F.Cu") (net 12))
 (segment (start 68.526 69.974) (end 68.526 65.476) (width 0.2) (layer "F.Cu") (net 12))
 (segment (start 76.74 54.795) (end 84.665 54.795) (width 0.2) (layer "F.Cu") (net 2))
 (segment (start 81.665 54.795) (end 81.74 54.72) (width 0.2) (layer "F.Cu") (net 2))
 (segment (start 81.24 54.795) (end 81.665 54.795) (width 0.2) (layer "F.Cu") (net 2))
 (segment (start 75.642 53.697) (end 76.74 54.795) (width 0.2) (layer "F.Cu") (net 2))
 (segment (start 84.665 54.795) (end 84.74 54.72) (width 0.2) (layer "F.Cu") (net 2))
 (segment (start 76.74 57.22) (end 76.74 54.795) (width 0.2) (layer "F.Cu") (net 2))
 (segment (start 71.576 53.697) (end 75.642 53.697) (width 0.2) (layer "F.Cu") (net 2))
 (segment (start 62.725 62.548) (end 71.576 53.697) (width 0.2) (layer "F.Cu") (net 2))
 (segment (start 62.725 70.05) (end 62.725 62.548) (width 0.2) (layer "F.Cu") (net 2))
 (segment (start 70.5 74.495) (end 70.5 59.8) (width 0.2) (layer "F.Cu") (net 6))
 (segment (start 71 81.995) (end 67 77.995) (width 0.2) (layer "F.Cu") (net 6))
 (segment (start 78 93) (end 71 86) (width 0.2) (layer "F.Cu") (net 6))
 (segment (start 70.5 59.8) (end 73 57.3) (width 0.2) (layer "F.Cu") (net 6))
 (segment (start 67 77.995) (end 70.5 74.495) (width 0.2) (layer "F.Cu") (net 6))
 (segment (start 78 92.98) (end 78 93) (width 0.2) (layer "F.Cu") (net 6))
 (segment (start 71 86) (end 71 81.995) (width 0.2) (layer "F.Cu") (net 6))
 (segment (start 100.5 42.81) (end 100.5 38.04) (width 0.2) (layer "F.Cu") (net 3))
 (segment (start 100.5 38.04) (end 96 33.54) (width 0.2) (layer "F.Cu") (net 3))
 (segment (start 96 43.04) (end 97.27 44.31) (width 0.2) (layer "F.Cu") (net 11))
 (segment (start 103.55 50.04) (end 104.551 49.039) (width 0.2) (layer "F.Cu") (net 11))
 (segment (start 97.27 44.31) (end 100.578484 44.31) (width 0.2) (layer "F.Cu") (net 11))
 (segment (start 102 46.639) (end 100.401 46.639) (width 0.2) (layer "F.Cu") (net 11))
 (segment (start 96 37.5) (end 96 43.04) (width 0.2) (layer "F.Cu") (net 11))
 (segment (start 104.551 49.039) (end 104.551 46.95484) (width 0.2) (layer "F.Cu") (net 11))
 (segment (start 104.551 46.95484) (end 104.23516 46.639) (width 0.2) (layer "F.Cu") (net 11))
 (segment (start 100.578484 44.31) (end 102 45.731516) (width 0.2) (layer "F.Cu") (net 11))
 (segment (start 102 45.731516) (end 102 46.639) (width 0.2) (layer "F.Cu") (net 11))
 (segment (start 100.401 46.639) (end 100 47.04) (width 0.2) (layer "F.Cu") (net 11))
 (segment (start 104.23516 46.639) (end 102 46.639) (width 0.2) (layer "F.Cu") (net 11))
 (segment (start 103.55 47.54) (end 101.51 49.58) (width 0.2) (layer "F.Cu") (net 10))
 (segment (start 101.51 49.58) (end 100 49.58) (width 0.2) (layer "F.Cu") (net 10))
 (segment (start 76.74 59.22) (end 77.74 59.22) (width 0.2) (layer "F.Cu") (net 5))
 (segment (start 77.74 59.22) (end 79.74 57.22) (width 0.2) (layer "F.Cu") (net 5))
 (segment (start 75 84.98) (end 75 56.76) (width 0.2) (layer "F.Cu") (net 37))
 (segment (start 75 56.76) (end 73 54.76) (width 0.2) (layer "F.Cu") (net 37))
 (segment (start 83 92.98) (end 75 84.98) (width 0.2) (layer "F.Cu") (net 37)))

